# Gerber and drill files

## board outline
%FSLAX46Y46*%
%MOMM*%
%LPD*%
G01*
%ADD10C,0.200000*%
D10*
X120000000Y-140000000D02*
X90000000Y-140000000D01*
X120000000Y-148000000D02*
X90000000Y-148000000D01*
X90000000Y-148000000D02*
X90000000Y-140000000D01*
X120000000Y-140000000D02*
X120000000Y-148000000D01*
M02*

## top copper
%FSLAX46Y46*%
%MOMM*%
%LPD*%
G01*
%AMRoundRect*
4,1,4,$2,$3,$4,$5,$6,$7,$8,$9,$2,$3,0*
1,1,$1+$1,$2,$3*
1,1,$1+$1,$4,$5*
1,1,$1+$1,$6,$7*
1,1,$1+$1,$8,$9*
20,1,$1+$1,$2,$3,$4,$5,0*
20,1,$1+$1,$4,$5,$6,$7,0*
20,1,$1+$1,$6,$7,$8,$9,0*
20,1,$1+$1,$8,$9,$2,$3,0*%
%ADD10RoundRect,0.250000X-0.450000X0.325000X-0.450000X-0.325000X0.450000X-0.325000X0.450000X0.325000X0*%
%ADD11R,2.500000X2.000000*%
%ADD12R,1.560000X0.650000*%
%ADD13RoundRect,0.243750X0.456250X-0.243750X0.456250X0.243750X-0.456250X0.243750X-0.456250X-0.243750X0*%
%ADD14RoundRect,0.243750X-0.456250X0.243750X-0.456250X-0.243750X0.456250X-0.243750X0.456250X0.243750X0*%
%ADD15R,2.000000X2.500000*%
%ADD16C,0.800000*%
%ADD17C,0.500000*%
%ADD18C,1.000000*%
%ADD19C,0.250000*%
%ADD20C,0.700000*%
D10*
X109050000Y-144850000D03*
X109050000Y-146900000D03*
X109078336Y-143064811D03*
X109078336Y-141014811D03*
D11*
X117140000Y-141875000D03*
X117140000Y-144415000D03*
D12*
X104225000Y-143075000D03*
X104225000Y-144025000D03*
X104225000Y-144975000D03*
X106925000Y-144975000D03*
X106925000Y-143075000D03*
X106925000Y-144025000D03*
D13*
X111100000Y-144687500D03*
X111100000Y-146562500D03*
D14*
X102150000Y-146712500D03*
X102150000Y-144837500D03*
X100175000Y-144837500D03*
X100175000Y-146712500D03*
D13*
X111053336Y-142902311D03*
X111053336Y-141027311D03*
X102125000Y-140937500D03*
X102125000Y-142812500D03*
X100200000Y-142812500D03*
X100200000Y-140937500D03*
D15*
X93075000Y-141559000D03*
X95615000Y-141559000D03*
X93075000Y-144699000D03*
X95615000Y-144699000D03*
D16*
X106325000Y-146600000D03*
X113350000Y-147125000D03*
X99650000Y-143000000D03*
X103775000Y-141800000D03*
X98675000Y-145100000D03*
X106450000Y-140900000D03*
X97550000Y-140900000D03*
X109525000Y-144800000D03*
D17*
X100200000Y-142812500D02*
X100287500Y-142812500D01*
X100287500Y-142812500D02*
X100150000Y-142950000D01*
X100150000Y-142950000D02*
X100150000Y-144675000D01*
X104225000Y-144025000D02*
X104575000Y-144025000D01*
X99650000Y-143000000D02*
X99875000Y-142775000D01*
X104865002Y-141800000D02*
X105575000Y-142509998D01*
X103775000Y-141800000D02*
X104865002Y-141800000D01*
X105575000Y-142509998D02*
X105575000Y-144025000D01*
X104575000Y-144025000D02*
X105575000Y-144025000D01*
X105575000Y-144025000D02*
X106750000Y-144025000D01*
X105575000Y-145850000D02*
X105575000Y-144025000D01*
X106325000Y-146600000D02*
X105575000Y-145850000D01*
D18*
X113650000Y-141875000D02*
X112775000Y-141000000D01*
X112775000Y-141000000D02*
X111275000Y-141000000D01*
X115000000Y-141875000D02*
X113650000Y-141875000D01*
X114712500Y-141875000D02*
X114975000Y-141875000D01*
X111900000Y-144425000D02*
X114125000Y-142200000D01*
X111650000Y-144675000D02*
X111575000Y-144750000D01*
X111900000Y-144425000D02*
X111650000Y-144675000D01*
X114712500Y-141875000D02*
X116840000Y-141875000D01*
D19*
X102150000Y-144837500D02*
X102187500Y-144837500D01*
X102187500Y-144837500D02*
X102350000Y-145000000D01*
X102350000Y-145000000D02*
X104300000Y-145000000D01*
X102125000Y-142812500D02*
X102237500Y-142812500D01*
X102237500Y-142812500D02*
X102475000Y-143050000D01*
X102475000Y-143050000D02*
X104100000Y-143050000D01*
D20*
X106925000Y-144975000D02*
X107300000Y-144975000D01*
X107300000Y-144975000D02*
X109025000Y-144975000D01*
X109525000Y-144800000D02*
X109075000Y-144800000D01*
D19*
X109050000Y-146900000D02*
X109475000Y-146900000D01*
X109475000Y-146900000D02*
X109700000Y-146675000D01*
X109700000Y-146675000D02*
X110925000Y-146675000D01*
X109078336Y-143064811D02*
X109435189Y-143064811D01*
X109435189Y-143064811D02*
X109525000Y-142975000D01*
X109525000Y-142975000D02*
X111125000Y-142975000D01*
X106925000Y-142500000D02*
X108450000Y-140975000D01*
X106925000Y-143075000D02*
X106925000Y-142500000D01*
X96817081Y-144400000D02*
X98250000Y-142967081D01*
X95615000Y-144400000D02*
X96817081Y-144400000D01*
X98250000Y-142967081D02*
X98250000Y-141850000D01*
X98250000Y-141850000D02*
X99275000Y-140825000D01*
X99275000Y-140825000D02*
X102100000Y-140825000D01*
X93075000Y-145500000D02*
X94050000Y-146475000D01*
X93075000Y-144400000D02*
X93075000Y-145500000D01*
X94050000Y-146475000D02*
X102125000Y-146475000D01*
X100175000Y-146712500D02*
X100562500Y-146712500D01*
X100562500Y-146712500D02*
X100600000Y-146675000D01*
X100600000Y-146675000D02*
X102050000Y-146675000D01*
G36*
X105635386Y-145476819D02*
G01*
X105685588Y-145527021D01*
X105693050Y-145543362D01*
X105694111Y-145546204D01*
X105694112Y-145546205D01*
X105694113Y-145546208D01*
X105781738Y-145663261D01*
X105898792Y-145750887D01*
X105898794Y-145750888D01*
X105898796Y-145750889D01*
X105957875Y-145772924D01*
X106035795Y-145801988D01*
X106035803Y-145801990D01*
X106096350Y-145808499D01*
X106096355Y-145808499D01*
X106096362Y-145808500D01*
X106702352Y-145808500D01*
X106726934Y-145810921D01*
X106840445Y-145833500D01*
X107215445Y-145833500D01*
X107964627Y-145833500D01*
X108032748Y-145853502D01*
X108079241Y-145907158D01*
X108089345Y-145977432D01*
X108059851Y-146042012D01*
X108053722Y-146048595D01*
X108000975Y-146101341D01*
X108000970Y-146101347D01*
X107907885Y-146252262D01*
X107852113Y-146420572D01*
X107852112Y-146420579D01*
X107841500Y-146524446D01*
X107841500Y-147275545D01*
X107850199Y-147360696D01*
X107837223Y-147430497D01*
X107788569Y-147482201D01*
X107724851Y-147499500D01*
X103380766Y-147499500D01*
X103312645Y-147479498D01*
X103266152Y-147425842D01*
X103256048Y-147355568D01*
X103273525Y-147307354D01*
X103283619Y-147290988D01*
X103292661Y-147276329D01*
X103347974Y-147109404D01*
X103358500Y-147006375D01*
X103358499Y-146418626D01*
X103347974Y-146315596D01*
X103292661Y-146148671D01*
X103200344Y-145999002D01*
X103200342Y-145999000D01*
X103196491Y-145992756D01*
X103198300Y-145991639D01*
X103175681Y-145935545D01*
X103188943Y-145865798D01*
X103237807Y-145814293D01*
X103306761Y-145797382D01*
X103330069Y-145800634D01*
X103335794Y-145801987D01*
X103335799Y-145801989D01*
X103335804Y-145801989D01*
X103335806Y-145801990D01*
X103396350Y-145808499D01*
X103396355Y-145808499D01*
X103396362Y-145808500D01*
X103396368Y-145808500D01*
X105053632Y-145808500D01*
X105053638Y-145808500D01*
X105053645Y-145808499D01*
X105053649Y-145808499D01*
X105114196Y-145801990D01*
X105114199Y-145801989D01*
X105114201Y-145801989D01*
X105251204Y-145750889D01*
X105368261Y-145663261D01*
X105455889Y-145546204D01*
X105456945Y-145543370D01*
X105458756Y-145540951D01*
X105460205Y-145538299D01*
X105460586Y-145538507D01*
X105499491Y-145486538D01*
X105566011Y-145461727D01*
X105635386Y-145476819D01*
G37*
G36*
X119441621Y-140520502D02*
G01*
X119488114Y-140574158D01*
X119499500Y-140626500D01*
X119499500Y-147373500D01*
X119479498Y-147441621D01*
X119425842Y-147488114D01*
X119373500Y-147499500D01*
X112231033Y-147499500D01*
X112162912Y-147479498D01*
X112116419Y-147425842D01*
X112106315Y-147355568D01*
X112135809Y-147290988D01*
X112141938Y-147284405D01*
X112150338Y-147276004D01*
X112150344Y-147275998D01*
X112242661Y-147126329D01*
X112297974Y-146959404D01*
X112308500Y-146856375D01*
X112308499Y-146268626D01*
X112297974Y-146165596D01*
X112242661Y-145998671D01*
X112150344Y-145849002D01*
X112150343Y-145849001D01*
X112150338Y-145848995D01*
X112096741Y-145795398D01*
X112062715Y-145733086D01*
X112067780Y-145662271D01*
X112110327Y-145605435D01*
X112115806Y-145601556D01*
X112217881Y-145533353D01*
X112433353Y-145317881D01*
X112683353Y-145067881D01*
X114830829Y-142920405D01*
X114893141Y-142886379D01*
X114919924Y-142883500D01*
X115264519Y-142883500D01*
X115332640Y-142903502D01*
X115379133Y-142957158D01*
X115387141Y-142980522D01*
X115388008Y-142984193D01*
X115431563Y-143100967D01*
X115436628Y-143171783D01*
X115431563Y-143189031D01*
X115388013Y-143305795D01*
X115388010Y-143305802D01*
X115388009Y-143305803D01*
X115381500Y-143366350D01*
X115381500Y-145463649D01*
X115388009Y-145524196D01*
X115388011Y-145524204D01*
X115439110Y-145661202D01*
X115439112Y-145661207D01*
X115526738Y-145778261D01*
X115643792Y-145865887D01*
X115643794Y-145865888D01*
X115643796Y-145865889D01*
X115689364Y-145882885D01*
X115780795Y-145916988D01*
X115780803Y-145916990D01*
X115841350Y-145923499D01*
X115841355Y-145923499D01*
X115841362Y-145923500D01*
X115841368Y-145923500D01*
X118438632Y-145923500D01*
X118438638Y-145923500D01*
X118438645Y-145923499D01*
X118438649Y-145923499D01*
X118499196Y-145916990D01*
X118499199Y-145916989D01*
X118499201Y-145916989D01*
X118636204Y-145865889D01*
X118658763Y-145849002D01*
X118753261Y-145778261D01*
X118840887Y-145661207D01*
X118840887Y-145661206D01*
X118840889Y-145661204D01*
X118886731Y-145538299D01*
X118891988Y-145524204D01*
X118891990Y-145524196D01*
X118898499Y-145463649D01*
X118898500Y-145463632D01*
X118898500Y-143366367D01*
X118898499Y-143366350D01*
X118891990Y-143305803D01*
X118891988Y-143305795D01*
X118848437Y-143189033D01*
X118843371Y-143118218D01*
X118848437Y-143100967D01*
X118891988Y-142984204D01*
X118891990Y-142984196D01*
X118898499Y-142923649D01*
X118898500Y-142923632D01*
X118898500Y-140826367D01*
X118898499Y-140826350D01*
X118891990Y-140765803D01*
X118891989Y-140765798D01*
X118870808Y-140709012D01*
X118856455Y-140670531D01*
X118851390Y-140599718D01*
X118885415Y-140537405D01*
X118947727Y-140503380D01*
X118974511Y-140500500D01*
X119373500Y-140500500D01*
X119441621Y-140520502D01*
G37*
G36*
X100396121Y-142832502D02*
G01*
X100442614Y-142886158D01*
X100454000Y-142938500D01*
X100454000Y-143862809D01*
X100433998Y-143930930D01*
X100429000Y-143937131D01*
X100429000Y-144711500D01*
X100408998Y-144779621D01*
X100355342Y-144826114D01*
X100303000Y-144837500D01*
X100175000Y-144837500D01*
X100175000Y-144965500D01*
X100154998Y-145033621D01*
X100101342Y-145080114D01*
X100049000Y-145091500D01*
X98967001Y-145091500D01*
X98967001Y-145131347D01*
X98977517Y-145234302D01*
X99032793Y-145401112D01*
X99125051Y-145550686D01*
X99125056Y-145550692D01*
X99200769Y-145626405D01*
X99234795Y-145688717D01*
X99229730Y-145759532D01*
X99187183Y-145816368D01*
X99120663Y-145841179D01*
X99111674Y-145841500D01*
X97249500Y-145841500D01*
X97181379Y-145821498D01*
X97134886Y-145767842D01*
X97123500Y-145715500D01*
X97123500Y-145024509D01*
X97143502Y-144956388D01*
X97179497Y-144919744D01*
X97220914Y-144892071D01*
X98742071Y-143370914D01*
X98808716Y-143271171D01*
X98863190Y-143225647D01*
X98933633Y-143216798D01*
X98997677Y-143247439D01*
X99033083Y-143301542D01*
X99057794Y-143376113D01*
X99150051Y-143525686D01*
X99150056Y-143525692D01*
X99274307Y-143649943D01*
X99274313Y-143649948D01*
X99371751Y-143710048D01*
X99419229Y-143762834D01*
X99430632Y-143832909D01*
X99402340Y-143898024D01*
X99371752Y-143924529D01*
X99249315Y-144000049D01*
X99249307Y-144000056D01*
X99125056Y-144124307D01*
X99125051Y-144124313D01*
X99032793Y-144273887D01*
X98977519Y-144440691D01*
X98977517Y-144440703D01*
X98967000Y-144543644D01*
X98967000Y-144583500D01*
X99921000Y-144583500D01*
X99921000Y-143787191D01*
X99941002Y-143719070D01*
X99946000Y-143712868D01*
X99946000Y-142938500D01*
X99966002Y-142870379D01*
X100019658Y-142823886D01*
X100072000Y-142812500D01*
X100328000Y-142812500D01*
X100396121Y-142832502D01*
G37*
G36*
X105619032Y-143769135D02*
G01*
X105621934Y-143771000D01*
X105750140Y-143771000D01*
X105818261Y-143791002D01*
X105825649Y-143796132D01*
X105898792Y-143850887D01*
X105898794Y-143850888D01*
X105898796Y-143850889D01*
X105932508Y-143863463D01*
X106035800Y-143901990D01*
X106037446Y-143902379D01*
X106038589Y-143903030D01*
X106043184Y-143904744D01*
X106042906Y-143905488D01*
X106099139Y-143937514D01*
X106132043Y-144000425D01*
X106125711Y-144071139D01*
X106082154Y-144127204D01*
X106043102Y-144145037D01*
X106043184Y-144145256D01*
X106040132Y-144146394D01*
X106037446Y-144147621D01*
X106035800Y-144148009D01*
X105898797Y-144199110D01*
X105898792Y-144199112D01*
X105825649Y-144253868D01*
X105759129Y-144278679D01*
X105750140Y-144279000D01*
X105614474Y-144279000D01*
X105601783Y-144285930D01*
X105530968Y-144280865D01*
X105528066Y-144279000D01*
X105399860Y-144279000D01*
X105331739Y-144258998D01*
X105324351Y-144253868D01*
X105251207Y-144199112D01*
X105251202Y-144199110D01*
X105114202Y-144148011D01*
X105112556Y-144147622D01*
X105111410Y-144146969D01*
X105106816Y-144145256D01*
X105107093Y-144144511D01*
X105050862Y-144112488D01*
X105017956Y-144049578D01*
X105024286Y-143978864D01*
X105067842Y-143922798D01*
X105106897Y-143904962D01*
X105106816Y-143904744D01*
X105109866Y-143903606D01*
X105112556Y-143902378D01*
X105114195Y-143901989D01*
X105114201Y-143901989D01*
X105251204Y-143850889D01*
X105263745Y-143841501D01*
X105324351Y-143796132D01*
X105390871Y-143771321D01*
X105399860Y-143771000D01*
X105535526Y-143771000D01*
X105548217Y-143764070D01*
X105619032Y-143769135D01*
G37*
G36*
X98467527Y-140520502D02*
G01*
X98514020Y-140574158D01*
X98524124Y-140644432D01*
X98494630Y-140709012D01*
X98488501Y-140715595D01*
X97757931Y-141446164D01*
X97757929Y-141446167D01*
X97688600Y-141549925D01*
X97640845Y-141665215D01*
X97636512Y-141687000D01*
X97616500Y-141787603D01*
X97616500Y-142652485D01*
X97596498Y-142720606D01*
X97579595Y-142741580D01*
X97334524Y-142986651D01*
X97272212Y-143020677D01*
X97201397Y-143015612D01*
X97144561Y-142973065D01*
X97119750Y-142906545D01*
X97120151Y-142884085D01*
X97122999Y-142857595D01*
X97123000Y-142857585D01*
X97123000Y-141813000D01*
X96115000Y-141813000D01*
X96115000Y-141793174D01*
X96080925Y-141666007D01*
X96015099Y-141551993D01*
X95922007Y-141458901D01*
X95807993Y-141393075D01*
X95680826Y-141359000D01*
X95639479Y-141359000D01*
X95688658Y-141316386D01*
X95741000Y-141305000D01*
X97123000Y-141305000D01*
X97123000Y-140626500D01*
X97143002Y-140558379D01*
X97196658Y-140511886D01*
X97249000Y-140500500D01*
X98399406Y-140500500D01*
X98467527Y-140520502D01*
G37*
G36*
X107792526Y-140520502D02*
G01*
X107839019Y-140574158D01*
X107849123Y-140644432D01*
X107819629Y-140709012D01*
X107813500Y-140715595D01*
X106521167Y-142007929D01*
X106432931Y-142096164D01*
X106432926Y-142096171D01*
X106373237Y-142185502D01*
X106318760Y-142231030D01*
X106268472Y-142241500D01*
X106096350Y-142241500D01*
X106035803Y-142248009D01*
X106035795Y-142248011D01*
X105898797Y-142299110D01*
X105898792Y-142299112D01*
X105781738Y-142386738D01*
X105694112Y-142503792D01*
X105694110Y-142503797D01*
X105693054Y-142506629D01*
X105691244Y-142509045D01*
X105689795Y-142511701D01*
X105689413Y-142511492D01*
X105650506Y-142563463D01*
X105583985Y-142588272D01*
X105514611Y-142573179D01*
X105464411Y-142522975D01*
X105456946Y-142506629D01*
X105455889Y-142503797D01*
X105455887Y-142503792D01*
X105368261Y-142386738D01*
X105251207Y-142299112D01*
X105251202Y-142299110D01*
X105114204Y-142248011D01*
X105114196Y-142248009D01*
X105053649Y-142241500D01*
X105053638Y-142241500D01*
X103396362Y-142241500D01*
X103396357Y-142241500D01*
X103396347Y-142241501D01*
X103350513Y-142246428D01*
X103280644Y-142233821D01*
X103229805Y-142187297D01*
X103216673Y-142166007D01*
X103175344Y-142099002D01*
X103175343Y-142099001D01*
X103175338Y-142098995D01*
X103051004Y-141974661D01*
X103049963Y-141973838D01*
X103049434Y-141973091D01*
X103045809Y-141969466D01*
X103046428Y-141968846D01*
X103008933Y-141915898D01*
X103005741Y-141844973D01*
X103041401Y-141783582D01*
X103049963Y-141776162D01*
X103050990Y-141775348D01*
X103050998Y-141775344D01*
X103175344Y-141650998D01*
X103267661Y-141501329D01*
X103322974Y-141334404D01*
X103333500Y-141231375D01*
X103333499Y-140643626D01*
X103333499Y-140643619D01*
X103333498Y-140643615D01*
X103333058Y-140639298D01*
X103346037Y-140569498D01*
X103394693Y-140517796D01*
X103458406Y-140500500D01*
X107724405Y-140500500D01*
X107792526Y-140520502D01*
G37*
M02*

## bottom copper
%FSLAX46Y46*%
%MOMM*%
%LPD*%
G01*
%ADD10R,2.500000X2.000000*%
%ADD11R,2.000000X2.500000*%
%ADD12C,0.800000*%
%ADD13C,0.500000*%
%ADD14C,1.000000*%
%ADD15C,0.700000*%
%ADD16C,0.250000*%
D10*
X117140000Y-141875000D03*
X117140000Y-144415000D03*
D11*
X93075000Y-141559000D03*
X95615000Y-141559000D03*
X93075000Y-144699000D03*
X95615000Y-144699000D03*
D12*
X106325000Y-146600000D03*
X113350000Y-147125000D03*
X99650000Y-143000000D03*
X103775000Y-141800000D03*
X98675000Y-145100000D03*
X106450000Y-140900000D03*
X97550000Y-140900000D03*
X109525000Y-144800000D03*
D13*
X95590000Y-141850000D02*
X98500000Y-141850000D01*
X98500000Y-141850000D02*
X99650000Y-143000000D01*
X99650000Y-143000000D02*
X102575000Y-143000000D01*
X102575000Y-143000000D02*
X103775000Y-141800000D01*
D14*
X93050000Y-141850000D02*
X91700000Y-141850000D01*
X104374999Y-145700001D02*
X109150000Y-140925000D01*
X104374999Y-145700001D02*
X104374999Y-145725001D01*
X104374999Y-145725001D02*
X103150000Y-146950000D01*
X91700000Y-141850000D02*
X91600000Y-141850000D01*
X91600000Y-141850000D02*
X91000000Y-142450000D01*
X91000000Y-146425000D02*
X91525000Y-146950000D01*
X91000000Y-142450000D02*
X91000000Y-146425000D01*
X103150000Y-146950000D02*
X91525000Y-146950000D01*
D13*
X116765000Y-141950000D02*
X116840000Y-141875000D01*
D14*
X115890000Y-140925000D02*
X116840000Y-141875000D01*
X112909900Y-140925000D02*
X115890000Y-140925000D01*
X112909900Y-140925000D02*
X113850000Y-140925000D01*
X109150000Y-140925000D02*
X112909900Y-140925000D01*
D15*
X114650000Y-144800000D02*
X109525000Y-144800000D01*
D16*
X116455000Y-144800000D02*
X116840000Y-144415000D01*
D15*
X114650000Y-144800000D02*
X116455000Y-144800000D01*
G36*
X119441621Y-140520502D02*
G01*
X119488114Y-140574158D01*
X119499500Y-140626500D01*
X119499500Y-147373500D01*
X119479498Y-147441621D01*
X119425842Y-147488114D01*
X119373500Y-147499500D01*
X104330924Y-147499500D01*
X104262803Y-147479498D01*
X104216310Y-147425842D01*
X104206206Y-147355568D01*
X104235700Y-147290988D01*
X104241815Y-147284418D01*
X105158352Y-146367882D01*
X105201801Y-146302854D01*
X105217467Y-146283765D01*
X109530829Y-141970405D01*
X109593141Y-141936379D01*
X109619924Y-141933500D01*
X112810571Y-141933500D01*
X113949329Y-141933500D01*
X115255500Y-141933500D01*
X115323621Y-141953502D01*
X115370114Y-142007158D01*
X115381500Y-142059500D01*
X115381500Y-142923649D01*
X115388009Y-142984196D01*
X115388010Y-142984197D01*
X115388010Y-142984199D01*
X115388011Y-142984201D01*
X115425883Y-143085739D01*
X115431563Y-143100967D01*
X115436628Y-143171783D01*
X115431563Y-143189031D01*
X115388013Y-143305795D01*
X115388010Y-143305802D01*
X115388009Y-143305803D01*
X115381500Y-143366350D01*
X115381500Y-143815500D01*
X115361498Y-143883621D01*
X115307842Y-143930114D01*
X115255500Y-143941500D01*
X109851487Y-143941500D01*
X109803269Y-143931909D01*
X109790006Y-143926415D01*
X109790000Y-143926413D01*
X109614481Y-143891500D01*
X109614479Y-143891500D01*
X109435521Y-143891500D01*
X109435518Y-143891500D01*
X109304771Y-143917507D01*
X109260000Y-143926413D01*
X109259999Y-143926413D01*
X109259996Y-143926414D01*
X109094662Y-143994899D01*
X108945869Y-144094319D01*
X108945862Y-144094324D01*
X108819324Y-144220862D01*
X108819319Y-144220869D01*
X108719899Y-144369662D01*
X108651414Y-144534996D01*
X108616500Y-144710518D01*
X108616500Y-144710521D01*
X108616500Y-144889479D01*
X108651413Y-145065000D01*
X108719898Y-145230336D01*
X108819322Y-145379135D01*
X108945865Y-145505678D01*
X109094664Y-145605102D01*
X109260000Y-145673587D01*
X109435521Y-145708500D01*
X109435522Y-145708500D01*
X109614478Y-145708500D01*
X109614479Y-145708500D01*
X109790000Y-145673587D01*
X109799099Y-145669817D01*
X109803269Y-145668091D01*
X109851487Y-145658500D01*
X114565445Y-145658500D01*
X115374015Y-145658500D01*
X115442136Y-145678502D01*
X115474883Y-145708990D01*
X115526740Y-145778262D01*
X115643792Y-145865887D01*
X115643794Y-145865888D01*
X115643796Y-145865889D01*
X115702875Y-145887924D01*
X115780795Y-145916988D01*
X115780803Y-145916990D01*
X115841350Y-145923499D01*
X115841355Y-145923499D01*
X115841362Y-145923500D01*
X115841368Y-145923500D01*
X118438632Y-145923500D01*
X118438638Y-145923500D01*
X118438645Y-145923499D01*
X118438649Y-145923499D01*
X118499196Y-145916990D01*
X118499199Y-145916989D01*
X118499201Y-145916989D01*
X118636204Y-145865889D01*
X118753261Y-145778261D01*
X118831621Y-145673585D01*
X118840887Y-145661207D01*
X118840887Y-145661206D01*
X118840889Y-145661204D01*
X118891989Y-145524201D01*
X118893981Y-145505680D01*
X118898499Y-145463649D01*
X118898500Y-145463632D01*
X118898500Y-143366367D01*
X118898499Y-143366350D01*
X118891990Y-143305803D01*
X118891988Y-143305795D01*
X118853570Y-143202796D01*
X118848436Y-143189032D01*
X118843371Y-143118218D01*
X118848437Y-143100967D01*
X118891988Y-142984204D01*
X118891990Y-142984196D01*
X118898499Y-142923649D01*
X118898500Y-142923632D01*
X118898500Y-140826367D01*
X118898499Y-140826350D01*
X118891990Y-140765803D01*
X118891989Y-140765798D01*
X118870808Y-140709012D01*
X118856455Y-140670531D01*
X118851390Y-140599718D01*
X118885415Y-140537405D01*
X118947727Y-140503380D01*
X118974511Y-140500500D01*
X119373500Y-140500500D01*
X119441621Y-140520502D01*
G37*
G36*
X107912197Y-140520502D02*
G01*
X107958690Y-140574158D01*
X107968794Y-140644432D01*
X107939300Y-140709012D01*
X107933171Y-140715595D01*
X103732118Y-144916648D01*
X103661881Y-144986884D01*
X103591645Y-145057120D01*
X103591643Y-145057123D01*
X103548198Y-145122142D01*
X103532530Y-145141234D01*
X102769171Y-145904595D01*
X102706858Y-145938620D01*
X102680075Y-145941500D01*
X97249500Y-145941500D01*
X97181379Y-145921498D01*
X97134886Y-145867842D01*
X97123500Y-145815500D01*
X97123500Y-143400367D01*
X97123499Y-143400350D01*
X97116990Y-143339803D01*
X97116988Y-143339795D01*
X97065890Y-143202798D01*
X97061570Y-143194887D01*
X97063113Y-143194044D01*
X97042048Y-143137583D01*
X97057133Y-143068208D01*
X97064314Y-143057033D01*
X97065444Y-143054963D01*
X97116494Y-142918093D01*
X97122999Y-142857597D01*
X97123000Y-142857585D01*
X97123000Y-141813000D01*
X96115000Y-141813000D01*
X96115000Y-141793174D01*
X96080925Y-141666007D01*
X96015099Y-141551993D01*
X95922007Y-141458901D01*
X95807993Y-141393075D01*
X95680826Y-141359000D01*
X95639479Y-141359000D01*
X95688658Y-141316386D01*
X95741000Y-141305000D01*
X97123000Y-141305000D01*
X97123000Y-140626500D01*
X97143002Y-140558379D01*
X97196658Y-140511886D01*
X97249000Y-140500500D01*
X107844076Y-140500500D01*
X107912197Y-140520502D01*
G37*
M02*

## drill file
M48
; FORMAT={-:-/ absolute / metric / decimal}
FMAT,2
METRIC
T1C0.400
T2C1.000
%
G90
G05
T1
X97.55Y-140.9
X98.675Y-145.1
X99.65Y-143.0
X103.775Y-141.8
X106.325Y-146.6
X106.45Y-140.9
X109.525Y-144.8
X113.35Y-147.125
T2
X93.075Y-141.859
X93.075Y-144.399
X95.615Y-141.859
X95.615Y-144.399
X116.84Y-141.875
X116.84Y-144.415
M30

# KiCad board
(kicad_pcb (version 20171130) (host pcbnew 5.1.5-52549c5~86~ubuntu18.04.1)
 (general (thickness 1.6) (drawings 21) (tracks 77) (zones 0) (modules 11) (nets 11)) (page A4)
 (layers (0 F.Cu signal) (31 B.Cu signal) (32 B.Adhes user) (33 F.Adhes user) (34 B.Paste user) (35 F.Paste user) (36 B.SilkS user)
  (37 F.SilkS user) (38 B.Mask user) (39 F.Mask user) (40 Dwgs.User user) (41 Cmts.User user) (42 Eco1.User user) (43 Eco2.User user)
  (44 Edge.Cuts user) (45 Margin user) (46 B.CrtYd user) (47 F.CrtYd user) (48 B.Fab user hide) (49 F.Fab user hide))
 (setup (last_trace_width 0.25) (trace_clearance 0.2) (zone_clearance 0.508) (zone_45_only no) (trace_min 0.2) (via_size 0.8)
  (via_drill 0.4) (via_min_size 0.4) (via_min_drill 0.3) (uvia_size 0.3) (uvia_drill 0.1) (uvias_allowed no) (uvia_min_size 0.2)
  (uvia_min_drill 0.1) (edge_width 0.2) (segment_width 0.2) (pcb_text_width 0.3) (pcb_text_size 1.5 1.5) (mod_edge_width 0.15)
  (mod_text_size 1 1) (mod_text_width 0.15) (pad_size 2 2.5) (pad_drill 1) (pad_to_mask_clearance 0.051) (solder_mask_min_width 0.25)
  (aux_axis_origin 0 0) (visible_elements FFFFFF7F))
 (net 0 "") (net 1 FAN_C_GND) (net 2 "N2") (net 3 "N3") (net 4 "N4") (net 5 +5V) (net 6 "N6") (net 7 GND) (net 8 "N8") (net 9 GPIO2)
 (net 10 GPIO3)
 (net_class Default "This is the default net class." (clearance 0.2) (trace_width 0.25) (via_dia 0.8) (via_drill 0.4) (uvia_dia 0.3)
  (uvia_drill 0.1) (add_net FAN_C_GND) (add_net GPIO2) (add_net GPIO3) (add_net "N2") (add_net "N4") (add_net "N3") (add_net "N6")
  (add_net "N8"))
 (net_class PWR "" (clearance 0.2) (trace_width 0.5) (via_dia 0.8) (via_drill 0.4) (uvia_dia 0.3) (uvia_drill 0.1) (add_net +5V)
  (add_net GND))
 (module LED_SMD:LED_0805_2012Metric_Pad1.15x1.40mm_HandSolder (layer F.Cu) (at 109.05 145.875 270)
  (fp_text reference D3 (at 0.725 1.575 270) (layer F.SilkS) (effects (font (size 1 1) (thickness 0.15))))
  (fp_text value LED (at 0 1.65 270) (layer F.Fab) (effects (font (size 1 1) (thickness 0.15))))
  (pad 1 smd roundrect (at -1.025 0 270) (size 1.15 1.4) (layers F.Cu F.Paste F.Mask) (roundrect_rratio 0.217391) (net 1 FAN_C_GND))
  (pad 2 smd roundrect (at 1.025 0 270) (size 1.15 1.4) (layers F.Cu F.Paste F.Mask) (roundrect_rratio 0.217391) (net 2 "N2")))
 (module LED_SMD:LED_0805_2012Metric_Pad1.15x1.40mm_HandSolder (layer F.Cu) (at 109.078336 142.039811 270)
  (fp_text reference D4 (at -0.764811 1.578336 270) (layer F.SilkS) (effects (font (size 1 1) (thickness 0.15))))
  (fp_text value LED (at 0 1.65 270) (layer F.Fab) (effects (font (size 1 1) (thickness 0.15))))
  (pad 2 smd roundrect (at 1.025 0 270) (size 1.15 1.4) (layers F.Cu F.Paste F.Mask) (roundrect_rratio 0.217391) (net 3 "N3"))
  (pad 1 smd roundrect (at -1.025 0 270) (size 1.15 1.4) (layers F.Cu F.Paste F.Mask) (roundrect_rratio 0.217391) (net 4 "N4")))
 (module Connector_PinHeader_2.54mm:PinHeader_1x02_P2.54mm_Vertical (layer F.Cu) (at 116.84 141.875)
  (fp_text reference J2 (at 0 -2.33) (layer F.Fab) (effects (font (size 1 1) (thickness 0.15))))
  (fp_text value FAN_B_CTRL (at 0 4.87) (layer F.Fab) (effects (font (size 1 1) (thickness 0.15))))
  (pad 1 thru_hole rect (at 0 0) (size 2.5 2) (drill 1 (offset 0.3 0)) (layers *.Cu *.Mask) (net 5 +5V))
  (pad 2 thru_hole rect (at 0 2.54) (size 2.5 2) (drill 1 (offset 0.3 0)) (layers *.Cu *.Mask) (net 1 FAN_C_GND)))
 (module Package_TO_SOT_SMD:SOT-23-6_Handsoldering (layer F.Cu) (at 105.575 144.025)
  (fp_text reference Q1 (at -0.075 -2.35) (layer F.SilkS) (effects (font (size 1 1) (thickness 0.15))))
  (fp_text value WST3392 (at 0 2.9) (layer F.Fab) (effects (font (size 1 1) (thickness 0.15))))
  (pad 1 smd rect (at -1.35 -0.95) (size 1.56 0.65) (layers F.Cu F.Paste F.Mask) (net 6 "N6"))
  (pad 2 smd rect (at -1.35 0) (size 1.56 0.65) (layers F.Cu F.Paste F.Mask) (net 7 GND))
  (pad 3 smd rect (at -1.35 0.95) (size 1.56 0.65) (layers F.Cu F.Paste F.Mask) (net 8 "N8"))
  (pad 4 smd rect (at 1.35 0.95) (size 1.56 0.65) (layers F.Cu F.Paste F.Mask) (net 1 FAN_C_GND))
  (pad 6 smd rect (at 1.35 -0.95) (size 1.56 0.65) (layers F.Cu F.Paste F.Mask) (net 4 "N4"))
  (pad 5 smd rect (at 1.35 0) (size 1.56 0.65) (layers F.Cu F.Paste F.Mask) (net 7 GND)))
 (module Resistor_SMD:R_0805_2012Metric (layer F.Cu) (at 111.1 145.625 90)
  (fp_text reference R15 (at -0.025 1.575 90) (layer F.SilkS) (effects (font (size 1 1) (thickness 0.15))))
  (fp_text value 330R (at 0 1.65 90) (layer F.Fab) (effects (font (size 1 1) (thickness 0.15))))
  (pad 2 smd roundrect (at 0.9375 0 90) (size 0.975 1.4) (layers F.Cu F.Paste F.Mask) (roundrect_rratio 0.25) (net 5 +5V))
  (pad 1 smd roundrect (at -0.9375 0 90) (size 0.975 1.4) (layers F.Cu F.Paste F.Mask) (roundrect_rratio 0.25) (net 2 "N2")))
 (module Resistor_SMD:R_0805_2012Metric (layer F.Cu) (at 102.15 145.775 270)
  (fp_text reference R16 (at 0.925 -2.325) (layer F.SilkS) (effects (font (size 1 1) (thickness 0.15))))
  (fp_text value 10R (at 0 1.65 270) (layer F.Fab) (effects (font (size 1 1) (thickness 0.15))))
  (pad 2 smd roundrect (at 0.9375 0 270) (size 0.975 1.4) (layers F.Cu F.Paste F.Mask) (roundrect_rratio 0.25) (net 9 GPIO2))
  (pad 1 smd roundrect (at -0.9375 0 270) (size 0.975 1.4) (layers F.Cu F.Paste F.Mask) (roundrect_rratio 0.25) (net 8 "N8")))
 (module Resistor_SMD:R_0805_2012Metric (layer F.Cu) (at 100.175 145.775 270)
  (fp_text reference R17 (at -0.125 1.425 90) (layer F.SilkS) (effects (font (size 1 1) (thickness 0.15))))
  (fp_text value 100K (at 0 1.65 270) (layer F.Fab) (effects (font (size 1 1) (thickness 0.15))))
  (pad 1 smd roundrect (at -0.9375 0 270) (size 0.975 1.4) (layers F.Cu F.Paste F.Mask) (roundrect_rratio 0.25) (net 7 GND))
  (pad 2 smd roundrect (at 0.9375 0 270) (size 0.975 1.4) (layers F.Cu F.Paste F.Mask) (roundrect_rratio 0.25) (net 9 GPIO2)))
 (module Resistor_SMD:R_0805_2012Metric (layer F.Cu) (at 111.053336 141.964811 90)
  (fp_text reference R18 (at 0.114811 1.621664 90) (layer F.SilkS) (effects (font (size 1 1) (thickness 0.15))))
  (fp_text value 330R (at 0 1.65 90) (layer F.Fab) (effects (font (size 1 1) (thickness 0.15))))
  (pad 1 smd roundrect (at -0.9375 0 90) (size 0.975 1.4) (layers F.Cu F.Paste F.Mask) (roundrect_rratio 0.25) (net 3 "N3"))
  (pad 2 smd roundrect (at 0.9375 0 90) (size 0.975 1.4) (layers F.Cu F.Paste F.Mask) (roundrect_rratio 0.25) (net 5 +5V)))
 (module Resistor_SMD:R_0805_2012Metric (layer F.Cu) (at 102.125 141.875 90)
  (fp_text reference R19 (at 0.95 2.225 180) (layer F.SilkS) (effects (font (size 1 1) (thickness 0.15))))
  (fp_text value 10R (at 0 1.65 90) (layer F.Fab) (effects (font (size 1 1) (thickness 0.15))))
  (pad 2 smd roundrect (at 0.9375 0 90) (size 0.975 1.4) (layers F.Cu F.Paste F.Mask) (roundrect_rratio 0.25) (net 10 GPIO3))
  (pad 1 smd roundrect (at -0.9375 0 90) (size 0.975 1.4) (layers F.Cu F.Paste F.Mask) (roundrect_rratio 0.25) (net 6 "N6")))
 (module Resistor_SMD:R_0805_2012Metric (layer F.Cu) (at 100.2 141.875 90)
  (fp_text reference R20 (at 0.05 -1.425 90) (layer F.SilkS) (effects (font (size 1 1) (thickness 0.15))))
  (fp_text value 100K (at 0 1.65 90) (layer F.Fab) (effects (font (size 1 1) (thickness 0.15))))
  (pad 1 smd roundrect (at -0.9375 0 90) (size 0.975 1.4) (layers F.Cu F.Paste F.Mask) (roundrect_rratio 0.25) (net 7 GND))
  (pad 2 smd roundrect (at 0.9375 0 90) (size 0.975 1.4) (layers F.Cu F.Paste F.Mask) (roundrect_rratio 0.25) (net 10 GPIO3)))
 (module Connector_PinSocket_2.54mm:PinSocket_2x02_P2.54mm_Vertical (layer B.Cu) (at 93.075 141.859 180)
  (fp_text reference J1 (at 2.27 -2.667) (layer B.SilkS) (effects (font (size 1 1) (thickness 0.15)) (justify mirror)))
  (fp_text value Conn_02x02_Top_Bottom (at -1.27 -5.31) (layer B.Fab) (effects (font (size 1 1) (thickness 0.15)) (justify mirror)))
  (pad 1 thru_hole rect (at 0 0 180) (size 2 2.5) (drill 1 (offset 0 0.3)) (layers *.Cu *.Mask) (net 5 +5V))
  (pad 2 thru_hole rect (at -2.54 0 180) (size 2 2.5) (drill 1 (offset 0 0.3)) (layers *.Cu *.Mask) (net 7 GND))
  (pad 3 thru_hole rect (at 0 -2.54 180) (size 2 2.5) (drill 1 (offset 0 -0.3)) (layers *.Cu *.Mask) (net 9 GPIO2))
  (pad 4 thru_hole rect (at -2.54 -2.54 180) (size 2 2.5) (drill 1 (offset 0 -0.3)) (layers *.Cu *.Mask) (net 10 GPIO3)))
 (gr_line (start 120 140) (end 90 140) (layer Edge.Cuts) (width 0.2))
 (gr_line (start 120 148) (end 90 148) (layer Edge.Cuts) (width 0.2))
 (gr_line (start 90 148) (end 90 140) (layer Edge.Cuts) (width 0.2))
 (gr_line (start 120 140) (end 120 148) (layer Edge.Cuts) (width 0.2))
 (via (at 106.325 146.6) (size 0.8) (drill 0.4) (layers F.Cu B.Cu) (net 7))
 (via (at 113.35 147.125) (size 0.8) (drill 0.4) (layers F.Cu B.Cu) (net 7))
 (segment (start 100.2 142.8125) (end 100.2875 142.8125) (width 0.5) (layer F.Cu) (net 7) (status 30))
 (segment (start 100.2875 142.8125) (end 100.15 142.95) (width 0.5) (layer F.Cu) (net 7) (status 30))
 (segment (start 100.15 142.95) (end 100.15 144.675) (width 0.5) (layer F.Cu) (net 7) (status 30))
 (segment (start 104.225 144.025) (end 104.575 144.025) (width 0.5) (layer F.Cu) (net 7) (status 30))
 (via (at 99.65 143) (size 0.8) (drill 0.4) (layers F.Cu B.Cu) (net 7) (status 30))
 (segment (start 95.59 141.85) (end 98.5 141.85) (width 0.5) (layer B.Cu) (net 7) (status 10))
 (segment (start 98.5 141.85) (end 99.65 143) (width 0.5) (layer B.Cu) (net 7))
 (segment (start 99.65 143) (end 99.875 142.775) (width 0.5) (layer F.Cu) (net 7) (status 30))
 (via (at 103.775 141.8) (size 0.8) (drill 0.4) (layers F.Cu B.Cu) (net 7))
 (segment (start 99.65 143) (end 102.575 143) (width 0.5) (layer B.Cu) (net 7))
 (segment (start 102.575 143) (end 103.775 141.8) (width 0.5) (layer B.Cu) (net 7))
 (segment (start 104.865002 141.8) (end 105.575 142.509998) (width 0.5) (layer F.Cu) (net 7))
 (segment (start 103.775 141.8) (end 104.865002 141.8) (width 0.5) (layer F.Cu) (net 7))
 (segment (start 105.575 142.509998) (end 105.575 144.025) (width 0.5) (layer F.Cu) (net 7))
 (segment (start 104.575 144.025) (end 105.575 144.025) (width 0.5) (layer F.Cu) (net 7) (status 10))
 (segment (start 105.575 144.025) (end 106.75 144.025) (width 0.5) (layer F.Cu) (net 7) (status 20))
 (via (at 98.675 145.1) (size 0.8) (drill 0.4) (layers F.Cu B.Cu) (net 7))
 (segment (start 105.575 145.85) (end 105.575 144.025) (width 0.5) (layer F.Cu) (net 7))
 (segment (start 106.325 146.6) (end 105.575 145.85) (width 0.5) (layer F.Cu) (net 7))
 (via (at 106.45 140.9) (size 0.8) (drill 0.4) (layers F.Cu B.Cu) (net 7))
 (via (at 97.55 140.9) (size 0.8) (drill 0.4) (layers F.Cu B.Cu) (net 7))
 (segment (start 93.05 141.85) (end 91.7 141.85) (width 1) (layer B.Cu) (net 5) (status 10))
 (segment (start 104.374999 145.700001) (end 109.15 140.925) (width 1) (layer B.Cu) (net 5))
 (segment (start 104.374999 145.700001) (end 104.374999 145.725001) (width 1) (layer B.Cu) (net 5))
 (segment (start 104.374999 145.725001) (end 103.15 146.95) (width 1) (layer B.Cu) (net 5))
 (segment (start 91.7 141.85) (end 91.6 141.85) (width 1) (layer B.Cu) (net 5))
 (segment (start 91.6 141.85) (end 91 142.45) (width 1) (layer B.Cu) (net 5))
 (segment (start 91 146.425) (end 91.525 146.95) (width 1) (layer B.Cu) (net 5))
 (segment (start 91 142.45) (end 91 146.425) (width 1) (layer B.Cu) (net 5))
 (segment (start 103.15 146.95) (end 91.525 146.95) (width 1) (layer B.Cu) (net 5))
 (segment (start 113.65 141.875) (end 112.775 141) (width 1) (layer F.Cu) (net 5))
 (segment (start 112.775 141) (end 111.275 141) (width 1) (layer F.Cu) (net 5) (status 20))
 (segment (start 115 141.875) (end 113.65 141.875) (width 1) (layer F.Cu) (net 5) (status 10))
 (segment (start 114.7125 141.875) (end 114.975 141.875) (width 1) (layer F.Cu) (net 5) (status 30))
 (segment (start 111.9 144.425) (end 114.125 142.2) (width 1) (layer F.Cu) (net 5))
 (segment (start 111.65 144.675) (end 111.575 144.75) (width 1) (layer F.Cu) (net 5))
 (segment (start 111.9 144.425) (end 111.65 144.675) (width 1) (layer F.Cu) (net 5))
 (segment (start 114.7125 141.875) (end 116.84 141.875) (width 1) (layer F.Cu) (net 5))
 (segment (start 116.765 141.95) (end 116.84 141.875) (width 0.5) (layer B.Cu) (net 5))
 (segment (start 115.89 140.925) (end 116.84 141.875) (width 1) (layer B.Cu) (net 5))
 (segment (start 112.9099 140.925) (end 115.89 140.925) (width 1) (layer B.Cu) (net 5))
 (segment (start 112.9099 140.925) (end 113.85 140.925) (width 1) (layer B.Cu) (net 5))
 (segment (start 109.15 140.925) (end 112.9099 140.925) (width 1) (layer B.Cu) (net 5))
 (segment (start 102.15 144.8375) (end 102.1875 144.8375) (width 0.25) (layer F.Cu) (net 8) (status 30))
 (segment (start 102.1875 144.8375) (end 102.35 145) (width 0.25) (layer F.Cu) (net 8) (status 30))
 (segment (start 102.35 145) (end 104.3 145) (width 0.25) (layer F.Cu) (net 8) (status 30))
 (segment (start 102.125 142.8125) (end 102.2375 142.8125) (width 0.25) (layer F.Cu) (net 6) (status 30))
 (segment (start 102.2375 142.8125) (end 102.475 143.05) (width 0.25) (layer F.Cu) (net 6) (status 30))
 (segment (start 102.475 143.05) (end 104.1 143.05) (width 0.25) (layer F.Cu) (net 6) (status 30))
 (segment (start 106.925 144.975) (end 107.3 144.975) (width 0.7) (layer F.Cu) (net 1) (status 30))
 (segment (start 107.3 144.975) (end 109.025 144.975) (width 0.7) (layer F.Cu) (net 1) (status 30))
 (via (at 109.525 144.8) (size 0.8) (drill 0.4) (layers F.Cu B.Cu) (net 1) (status 30))
 (segment (start 114.65 144.8) (end 109.525 144.8) (width 0.7) (layer B.Cu) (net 1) (status 10))
 (segment (start 109.525 144.8) (end 109.075 144.8) (width 0.7) (layer F.Cu) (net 1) (status 30))
 (segment (start 116.455 144.8) (end 116.84 144.415) (width 0.25) (layer B.Cu) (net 1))
 (segment (start 114.65 144.8) (end 116.455 144.8) (width 0.7) (layer B.Cu) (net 1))
 (segment (start 109.05 146.9) (end 109.475 146.9) (width 0.25) (layer F.Cu) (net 2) (status 30))
 (segment (start 109.475 146.9) (end 109.7 146.675) (width 0.25) (layer F.Cu) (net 2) (status 30))
 (segment (start 109.7 146.675) (end 110.925 146.675) (width 0.25) (layer F.Cu) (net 2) (status 30))
 (segment (start 109.078336 143.064811) (end 109.435189 143.064811) (width 0.25) (layer F.Cu) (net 3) (status 30))
 (segment (start 109.435189 143.064811) (end 109.525 142.975) (width 0.25) (layer F.Cu) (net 3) (status 30))
 (segment (start 109.525 142.975) (end 111.125 142.975) (width 0.25) (layer F.Cu) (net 3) (status 30))
 (segment (start 106.925 142.5) (end 108.45 140.975) (width 0.25) (layer F.Cu) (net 4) (status 20))
 (segment (start 106.925 143.075) (end 106.925 142.5) (width 0.25) (layer F.Cu) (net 4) (status 10))
 (segment (start 96.817081 144.4) (end 98.25 142.967081) (width 0.25) (layer F.Cu) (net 10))
 (segment (start 95.615 144.4) (end 96.817081 144.4) (width 0.25) (layer F.Cu) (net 10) (status 10))
 (segment (start 98.25 142.967081) (end 98.25 141.85) (width 0.25) (layer F.Cu) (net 10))
 (segment (start 98.25 141.85) (end 99.275 140.825) (width 0.25) (layer F.Cu) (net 10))
 (segment (start 99.275 140.825) (end 102.1 140.825) (width 0.25) (layer F.Cu) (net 10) (status 20))
 (segment (start 93.075 145.5) (end 94.05 146.475) (width 0.25) (layer F.Cu) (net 9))
 (segment (start 93.075 144.4) (end 93.075 145.5) (width 0.25) (layer F.Cu) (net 9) (status 10))
 (segment (start 94.05 146.475) (end 102.125 146.475) (width 0.25) (layer F.Cu) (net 9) (status 20))
 (segment (start 100.175 146.7125) (end 100.5625 146.7125) (width 0.25) (layer F.Cu) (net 9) (status 30))
 (segment (start 100.5625 146.7125) (end 100.6 146.675) (width 0.25) (layer F.Cu) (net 9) (status 30))
 (segment (start 100.6 146.675) (end 102.05 146.675) (width 0.25) (layer F.Cu) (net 9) (status 30))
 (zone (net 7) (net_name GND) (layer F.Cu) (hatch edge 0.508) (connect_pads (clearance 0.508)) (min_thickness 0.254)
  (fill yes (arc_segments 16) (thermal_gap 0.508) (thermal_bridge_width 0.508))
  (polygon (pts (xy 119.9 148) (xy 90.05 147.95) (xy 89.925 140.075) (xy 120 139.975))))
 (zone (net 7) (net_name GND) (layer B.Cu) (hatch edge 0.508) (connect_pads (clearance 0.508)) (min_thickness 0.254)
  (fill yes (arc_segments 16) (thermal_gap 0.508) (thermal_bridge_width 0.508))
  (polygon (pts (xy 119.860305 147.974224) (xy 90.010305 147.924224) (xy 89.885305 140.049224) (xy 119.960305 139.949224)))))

